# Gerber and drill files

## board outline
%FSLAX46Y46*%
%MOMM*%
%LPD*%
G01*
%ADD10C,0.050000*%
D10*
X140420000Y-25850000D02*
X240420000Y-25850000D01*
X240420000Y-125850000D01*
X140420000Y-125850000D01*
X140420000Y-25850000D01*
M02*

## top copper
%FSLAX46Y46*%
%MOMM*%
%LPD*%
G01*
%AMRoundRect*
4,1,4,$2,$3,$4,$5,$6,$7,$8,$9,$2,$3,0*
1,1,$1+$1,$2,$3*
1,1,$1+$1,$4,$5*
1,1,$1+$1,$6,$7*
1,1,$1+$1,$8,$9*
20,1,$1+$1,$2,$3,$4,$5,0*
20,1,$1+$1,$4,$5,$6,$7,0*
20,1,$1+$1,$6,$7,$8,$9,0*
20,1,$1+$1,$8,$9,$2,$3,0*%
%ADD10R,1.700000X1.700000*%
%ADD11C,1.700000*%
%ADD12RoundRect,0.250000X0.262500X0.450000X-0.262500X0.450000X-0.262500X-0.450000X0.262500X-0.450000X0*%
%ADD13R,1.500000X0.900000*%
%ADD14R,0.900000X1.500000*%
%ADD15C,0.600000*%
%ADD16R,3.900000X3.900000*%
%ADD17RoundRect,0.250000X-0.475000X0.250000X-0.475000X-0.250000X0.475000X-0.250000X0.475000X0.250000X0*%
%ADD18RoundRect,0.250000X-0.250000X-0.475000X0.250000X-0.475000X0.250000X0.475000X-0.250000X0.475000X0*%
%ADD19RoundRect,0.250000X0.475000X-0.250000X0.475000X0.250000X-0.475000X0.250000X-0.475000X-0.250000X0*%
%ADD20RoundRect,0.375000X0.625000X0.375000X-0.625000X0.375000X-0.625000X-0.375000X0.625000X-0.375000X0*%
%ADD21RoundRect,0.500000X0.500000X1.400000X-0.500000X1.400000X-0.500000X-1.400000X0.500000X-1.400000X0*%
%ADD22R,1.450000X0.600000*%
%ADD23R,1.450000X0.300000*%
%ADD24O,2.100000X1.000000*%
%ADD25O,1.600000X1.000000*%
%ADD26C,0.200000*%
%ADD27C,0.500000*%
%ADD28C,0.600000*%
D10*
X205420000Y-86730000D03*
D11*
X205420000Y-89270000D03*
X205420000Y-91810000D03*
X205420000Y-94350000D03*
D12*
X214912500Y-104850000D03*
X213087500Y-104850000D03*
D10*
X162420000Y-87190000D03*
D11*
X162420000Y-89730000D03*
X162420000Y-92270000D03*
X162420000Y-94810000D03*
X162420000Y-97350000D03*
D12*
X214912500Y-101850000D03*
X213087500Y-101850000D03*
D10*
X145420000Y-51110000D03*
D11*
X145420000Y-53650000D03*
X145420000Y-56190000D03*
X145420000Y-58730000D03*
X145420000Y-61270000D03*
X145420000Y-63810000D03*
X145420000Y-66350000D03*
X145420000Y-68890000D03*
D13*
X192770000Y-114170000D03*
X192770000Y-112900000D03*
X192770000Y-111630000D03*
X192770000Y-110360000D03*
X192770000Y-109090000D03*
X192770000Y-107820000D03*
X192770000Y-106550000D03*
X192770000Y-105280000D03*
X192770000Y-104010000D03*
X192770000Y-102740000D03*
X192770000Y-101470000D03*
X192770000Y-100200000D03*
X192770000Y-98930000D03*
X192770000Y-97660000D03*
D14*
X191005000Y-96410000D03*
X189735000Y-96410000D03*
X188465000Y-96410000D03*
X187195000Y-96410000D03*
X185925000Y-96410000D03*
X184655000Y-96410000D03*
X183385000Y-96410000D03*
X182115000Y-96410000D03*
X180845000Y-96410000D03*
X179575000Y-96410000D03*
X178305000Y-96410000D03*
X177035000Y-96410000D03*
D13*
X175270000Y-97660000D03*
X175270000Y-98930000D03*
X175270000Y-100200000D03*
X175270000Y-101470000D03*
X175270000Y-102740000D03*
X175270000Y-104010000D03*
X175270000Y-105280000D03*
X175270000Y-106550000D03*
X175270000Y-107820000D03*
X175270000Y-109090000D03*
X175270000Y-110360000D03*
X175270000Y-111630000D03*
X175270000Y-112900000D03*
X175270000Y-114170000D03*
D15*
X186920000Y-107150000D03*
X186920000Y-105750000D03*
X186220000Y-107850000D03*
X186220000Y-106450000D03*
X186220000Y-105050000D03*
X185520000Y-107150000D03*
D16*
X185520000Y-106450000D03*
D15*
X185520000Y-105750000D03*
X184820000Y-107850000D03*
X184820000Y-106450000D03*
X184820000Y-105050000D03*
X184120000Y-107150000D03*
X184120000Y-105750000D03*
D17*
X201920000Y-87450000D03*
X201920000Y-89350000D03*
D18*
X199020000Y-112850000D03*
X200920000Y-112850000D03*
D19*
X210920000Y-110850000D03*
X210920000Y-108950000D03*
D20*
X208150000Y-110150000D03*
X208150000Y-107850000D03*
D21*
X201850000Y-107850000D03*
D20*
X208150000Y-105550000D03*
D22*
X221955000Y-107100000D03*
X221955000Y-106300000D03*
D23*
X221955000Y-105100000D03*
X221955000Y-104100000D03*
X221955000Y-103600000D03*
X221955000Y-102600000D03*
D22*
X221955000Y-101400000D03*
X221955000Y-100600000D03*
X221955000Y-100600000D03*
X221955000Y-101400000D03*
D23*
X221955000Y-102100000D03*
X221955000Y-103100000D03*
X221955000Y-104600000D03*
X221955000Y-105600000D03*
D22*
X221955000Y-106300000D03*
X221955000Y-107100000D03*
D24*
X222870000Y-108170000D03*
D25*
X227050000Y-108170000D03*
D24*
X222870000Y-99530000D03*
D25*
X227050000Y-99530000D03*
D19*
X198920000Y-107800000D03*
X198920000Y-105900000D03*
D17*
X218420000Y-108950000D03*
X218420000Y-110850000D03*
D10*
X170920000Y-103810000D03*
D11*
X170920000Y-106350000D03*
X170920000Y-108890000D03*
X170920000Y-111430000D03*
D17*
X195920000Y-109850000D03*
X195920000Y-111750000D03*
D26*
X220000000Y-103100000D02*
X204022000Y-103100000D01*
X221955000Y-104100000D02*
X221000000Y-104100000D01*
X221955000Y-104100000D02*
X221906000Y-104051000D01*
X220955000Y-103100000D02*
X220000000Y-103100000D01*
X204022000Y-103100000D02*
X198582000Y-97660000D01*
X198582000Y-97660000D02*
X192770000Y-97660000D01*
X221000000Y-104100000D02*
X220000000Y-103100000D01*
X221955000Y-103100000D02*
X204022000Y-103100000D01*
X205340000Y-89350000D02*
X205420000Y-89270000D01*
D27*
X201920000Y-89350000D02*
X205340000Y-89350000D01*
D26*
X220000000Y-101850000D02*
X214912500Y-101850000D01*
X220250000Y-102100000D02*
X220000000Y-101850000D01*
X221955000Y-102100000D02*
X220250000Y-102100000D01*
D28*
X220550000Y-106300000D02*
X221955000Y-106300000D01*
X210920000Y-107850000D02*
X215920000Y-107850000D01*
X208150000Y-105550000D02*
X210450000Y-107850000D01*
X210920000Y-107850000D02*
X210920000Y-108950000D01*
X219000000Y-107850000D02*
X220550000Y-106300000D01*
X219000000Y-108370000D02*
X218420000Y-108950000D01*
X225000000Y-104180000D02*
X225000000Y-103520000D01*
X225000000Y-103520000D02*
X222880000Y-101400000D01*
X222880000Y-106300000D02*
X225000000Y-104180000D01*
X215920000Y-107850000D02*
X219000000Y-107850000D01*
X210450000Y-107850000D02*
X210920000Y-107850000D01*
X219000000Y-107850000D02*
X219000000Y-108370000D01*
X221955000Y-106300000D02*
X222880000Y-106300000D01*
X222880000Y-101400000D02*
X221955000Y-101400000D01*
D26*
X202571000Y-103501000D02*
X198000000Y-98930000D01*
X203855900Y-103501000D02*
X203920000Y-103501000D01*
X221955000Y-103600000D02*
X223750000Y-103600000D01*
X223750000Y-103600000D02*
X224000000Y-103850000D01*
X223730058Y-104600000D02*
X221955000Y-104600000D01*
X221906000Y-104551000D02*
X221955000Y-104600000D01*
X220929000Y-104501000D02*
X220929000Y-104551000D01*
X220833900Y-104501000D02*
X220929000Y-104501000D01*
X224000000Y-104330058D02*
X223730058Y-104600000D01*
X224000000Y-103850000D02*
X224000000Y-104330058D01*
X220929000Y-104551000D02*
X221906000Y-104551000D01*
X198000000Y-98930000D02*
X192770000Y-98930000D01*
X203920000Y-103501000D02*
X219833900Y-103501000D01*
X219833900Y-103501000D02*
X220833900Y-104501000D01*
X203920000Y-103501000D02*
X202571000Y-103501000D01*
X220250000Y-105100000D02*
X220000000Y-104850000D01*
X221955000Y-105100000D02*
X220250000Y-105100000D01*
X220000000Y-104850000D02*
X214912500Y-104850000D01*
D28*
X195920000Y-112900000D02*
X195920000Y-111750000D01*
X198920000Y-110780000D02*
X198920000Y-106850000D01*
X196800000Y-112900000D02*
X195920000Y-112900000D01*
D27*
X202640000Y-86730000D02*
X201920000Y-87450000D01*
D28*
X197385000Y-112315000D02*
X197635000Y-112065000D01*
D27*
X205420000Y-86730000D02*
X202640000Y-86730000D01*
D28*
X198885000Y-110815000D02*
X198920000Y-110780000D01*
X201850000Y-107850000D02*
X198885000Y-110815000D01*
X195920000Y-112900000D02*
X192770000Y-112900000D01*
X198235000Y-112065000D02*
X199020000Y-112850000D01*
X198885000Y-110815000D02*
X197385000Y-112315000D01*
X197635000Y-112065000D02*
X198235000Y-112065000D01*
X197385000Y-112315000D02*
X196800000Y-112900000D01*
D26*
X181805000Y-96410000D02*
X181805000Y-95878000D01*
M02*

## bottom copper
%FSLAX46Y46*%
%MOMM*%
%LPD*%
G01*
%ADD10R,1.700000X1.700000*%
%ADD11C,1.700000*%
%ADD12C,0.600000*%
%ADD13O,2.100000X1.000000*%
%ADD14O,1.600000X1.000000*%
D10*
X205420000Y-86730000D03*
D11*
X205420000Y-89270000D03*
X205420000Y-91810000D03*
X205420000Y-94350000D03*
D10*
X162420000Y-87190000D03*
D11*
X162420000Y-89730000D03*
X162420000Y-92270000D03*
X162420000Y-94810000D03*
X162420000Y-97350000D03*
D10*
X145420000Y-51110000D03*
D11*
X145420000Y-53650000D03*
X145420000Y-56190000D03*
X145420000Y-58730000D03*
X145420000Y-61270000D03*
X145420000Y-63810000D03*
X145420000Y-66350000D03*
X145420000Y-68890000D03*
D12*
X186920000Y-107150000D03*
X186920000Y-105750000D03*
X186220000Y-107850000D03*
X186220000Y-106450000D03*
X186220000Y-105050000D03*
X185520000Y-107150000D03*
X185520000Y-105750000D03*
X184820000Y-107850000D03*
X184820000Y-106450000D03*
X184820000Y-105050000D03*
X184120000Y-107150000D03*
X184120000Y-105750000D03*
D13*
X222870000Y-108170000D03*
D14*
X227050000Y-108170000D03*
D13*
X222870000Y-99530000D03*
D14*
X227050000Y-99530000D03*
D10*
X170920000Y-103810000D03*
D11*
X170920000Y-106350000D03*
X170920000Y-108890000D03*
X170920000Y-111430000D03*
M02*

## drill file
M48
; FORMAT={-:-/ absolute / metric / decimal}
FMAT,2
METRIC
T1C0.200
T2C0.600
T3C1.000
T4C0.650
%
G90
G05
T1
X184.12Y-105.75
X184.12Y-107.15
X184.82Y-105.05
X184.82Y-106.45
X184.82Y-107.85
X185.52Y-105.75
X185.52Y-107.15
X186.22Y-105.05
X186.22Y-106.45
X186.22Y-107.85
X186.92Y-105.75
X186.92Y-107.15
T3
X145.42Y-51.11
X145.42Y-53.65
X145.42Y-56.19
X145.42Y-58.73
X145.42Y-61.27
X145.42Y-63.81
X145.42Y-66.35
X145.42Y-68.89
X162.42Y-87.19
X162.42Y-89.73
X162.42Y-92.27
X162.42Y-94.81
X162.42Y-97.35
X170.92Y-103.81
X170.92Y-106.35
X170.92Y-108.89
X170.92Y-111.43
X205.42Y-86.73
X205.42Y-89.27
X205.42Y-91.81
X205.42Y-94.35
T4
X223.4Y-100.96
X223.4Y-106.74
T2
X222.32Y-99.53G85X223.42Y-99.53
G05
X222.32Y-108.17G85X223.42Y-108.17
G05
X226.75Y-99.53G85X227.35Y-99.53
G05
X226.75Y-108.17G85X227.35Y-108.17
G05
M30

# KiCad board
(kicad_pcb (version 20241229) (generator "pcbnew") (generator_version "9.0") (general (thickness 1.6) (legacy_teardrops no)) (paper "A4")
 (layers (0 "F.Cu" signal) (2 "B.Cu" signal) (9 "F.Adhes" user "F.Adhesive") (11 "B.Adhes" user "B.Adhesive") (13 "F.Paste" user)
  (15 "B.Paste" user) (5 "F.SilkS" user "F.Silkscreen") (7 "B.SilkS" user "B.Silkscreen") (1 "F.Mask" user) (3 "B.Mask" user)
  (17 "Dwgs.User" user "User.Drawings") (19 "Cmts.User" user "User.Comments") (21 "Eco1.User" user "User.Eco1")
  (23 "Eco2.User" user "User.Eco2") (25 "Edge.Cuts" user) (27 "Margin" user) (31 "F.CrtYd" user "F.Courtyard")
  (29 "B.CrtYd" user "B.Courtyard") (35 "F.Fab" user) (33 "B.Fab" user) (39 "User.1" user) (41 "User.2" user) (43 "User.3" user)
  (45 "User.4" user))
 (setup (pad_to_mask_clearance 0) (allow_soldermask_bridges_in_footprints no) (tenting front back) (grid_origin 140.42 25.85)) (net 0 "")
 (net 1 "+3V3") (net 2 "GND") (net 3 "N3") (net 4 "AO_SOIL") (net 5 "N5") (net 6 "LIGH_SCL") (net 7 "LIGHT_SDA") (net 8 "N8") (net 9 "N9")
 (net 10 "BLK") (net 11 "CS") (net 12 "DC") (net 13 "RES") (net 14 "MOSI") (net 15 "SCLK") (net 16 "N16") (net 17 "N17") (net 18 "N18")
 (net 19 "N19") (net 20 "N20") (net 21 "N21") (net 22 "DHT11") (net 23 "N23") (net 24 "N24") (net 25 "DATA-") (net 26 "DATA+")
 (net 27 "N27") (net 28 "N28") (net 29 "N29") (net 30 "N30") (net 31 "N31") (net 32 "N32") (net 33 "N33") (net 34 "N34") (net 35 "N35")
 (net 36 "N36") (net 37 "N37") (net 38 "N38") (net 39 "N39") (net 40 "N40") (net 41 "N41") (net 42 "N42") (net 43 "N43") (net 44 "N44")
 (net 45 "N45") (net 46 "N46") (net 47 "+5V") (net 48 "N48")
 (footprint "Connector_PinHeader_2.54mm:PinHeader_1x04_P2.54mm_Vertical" (layer "F.Cu") (at 205.42 86.73)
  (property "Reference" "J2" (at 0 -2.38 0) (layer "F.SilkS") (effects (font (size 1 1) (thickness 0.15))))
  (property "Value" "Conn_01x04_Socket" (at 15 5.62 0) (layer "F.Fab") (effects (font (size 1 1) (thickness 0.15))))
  (pad "1" thru_hole rect (at 0 0) (size 1.7 1.7) (drill 1) (layers "*.Cu" "*.Mask") (remove_unused_layers no) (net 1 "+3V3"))
  (pad "2" thru_hole circle (at 0 2.54) (size 1.7 1.7) (drill 1) (layers "*.Cu" "*.Mask") (remove_unused_layers no) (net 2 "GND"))
  (pad "3" thru_hole circle (at 0 5.08) (size 1.7 1.7) (drill 1) (layers "*.Cu" "*.Mask") (remove_unused_layers no) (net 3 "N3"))
  (pad "4" thru_hole circle (at 0 7.62) (size 1.7 1.7) (drill 1) (layers "*.Cu" "*.Mask") (remove_unused_layers no) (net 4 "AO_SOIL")))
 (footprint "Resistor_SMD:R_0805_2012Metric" (layer "F.Cu") (at 214 104.85 180)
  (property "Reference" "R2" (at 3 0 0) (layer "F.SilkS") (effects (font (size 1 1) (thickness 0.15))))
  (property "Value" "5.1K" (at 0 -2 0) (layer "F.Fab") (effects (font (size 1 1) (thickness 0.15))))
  (pad "1" smd roundrect (at -0.9125 0 180) (size 1.025 1.4) (layers "F.Cu" "F.Mask" "F.Paste") (roundrect_rratio 0.243902) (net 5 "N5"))
  (pad "2" smd roundrect (at 0.9125 0 180) (size 1.025 1.4) (layers "F.Cu" "F.Mask" "F.Paste") (roundrect_rratio 0.243902) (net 2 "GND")))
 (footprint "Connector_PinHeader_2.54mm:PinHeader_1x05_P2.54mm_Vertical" (layer "F.Cu") (at 162.42 87.19)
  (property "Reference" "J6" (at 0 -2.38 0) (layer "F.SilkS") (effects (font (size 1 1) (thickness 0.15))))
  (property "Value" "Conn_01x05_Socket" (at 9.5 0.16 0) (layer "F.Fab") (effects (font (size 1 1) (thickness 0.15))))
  (pad "1" thru_hole rect (at 0 0) (size 1.7 1.7) (drill 1) (layers "*.Cu" "*.Mask") (remove_unused_layers no) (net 1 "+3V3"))
  (pad "2" thru_hole circle (at 0 2.54) (size 1.7 1.7) (drill 1) (layers "*.Cu" "*.Mask") (remove_unused_layers no) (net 2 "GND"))
  (pad "3" thru_hole circle (at 0 5.08) (size 1.7 1.7) (drill 1) (layers "*.Cu" "*.Mask") (remove_unused_layers no) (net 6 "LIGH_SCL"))
  (pad "4" thru_hole circle (at 0 7.62) (size 1.7 1.7) (drill 1) (layers "*.Cu" "*.Mask") (remove_unused_layers no) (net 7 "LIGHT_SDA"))
  (pad "5" thru_hole circle (at 0 10.16) (size 1.7 1.7) (drill 1) (layers "*.Cu" "*.Mask") (remove_unused_layers no) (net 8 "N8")))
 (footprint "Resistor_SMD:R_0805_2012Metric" (layer "F.Cu") (at 214 101.85 180)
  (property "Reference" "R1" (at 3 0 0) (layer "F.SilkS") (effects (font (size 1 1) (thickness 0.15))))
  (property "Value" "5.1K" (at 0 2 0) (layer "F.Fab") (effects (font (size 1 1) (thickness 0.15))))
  (pad "1" smd roundrect (at -0.9125 0 180) (size 1.025 1.4) (layers "F.Cu" "F.Mask" "F.Paste") (roundrect_rratio 0.243902) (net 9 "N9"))
  (pad "2" smd roundrect (at 0.9125 0 180) (size 1.025 1.4) (layers "F.Cu" "F.Mask" "F.Paste") (roundrect_rratio 0.243902) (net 2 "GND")))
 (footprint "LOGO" (layer "F.Cu") (at 224.5 115)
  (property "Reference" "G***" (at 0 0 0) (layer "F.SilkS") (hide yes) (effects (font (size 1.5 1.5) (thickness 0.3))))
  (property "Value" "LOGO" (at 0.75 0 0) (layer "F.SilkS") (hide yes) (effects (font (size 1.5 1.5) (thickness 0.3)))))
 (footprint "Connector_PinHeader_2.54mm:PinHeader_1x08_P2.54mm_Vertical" (layer "F.Cu") (at 145.42 51.11)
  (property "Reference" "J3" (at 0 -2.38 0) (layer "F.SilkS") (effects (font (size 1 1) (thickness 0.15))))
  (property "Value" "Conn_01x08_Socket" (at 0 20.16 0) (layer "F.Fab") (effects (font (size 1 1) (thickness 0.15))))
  (pad "1" thru_hole rect (at 0 0) (size 1.7 1.7) (drill 1) (layers "*.Cu" "*.Mask") (remove_unused_layers no) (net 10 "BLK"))
  (pad "2" thru_hole circle (at 0 2.54) (size 1.7 1.7) (drill 1) (layers "*.Cu" "*.Mask") (remove_unused_layers no) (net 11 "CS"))
  (pad "3" thru_hole circle (at 0 5.08) (size 1.7 1.7) (drill 1) (layers "*.Cu" "*.Mask") (remove_unused_layers no) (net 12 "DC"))
  (pad "4" thru_hole circle (at 0 7.62) (size 1.7 1.7) (drill 1) (layers "*.Cu" "*.Mask") (remove_unused_layers no) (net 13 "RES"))
  (pad "5" thru_hole circle (at 0 10.16) (size 1.7 1.7) (drill 1) (layers "*.Cu" "*.Mask") (remove_unused_layers no) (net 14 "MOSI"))
  (pad "6" thru_hole circle (at 0 12.7) (size 1.7 1.7) (drill 1) (layers "*.Cu" "*.Mask") (remove_unused_layers no) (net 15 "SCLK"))
  (pad "7" thru_hole circle (at 0 15.24) (size 1.7 1.7) (drill 1) (layers "*.Cu" "*.Mask") (remove_unused_layers no) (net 1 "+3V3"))
  (pad "8" thru_hole circle (at 0 17.78) (size 1.7 1.7) (drill 1) (layers "*.Cu" "*.Mask") (remove_unused_layers no) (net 2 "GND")))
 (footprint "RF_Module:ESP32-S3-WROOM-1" (layer "F.Cu") (at 184.02 108.91 180)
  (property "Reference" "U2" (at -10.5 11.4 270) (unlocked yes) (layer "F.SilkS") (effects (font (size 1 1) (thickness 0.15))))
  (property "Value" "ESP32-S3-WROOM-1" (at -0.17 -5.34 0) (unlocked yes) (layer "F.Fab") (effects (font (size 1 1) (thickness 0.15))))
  (pad "" smd rect (at -2.9 1.06 180) (size 0.9 0.9) (layers "F.Paste"))
  (pad "" smd rect (at -2.9 2.46 90) (size 0.9 0.9) (layers "F.Paste"))
  (pad "" smd rect (at -2.9 3.86 180) (size 0.9 0.9) (layers "F.Paste"))
  (pad "" smd rect (at -1.5 1.06 90) (size 0.9 0.9) (layers "F.Paste"))
  (pad "" smd rect (at -1.5 2.46 90) (size 0.9 0.9) (layers "F.Paste"))
  (pad "" smd rect (at -1.5 3.86 90) (size 0.9 0.9) (layers "F.Paste"))
  (pad "" smd rect (at -0.1 1.06 90) (size 0.9 0.9) (layers "F.Paste"))
  (pad "" smd rect (at -0.1 2.46 90) (size 0.9 0.9) (layers "F.Paste"))
  (pad "" smd rect (at -0.1 3.86 90) (size 0.9 0.9) (layers "F.Paste"))
  (pad "1" smd rect (at -8.75 -5.26 180) (size 1.5 0.9) (layers "F.Cu" "F.Mask" "F.Paste") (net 2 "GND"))
  (pad "2" smd rect (at -8.75 -3.99 180) (size 1.5 0.9) (layers "F.Cu" "F.Mask" "F.Paste") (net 1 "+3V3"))
  (pad "3" smd rect (at -8.75 -2.72 180) (size 1.5 0.9) (layers "F.Cu" "F.Mask" "F.Paste") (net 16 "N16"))
  (pad "4" smd rect (at -8.75 -1.45 180) (size 1.5 0.9) (layers "F.Cu" "F.Mask" "F.Paste") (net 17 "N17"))
  (pad "5" smd rect (at -8.75 -0.18 180) (size 1.5 0.9) (layers "F.Cu" "F.Mask" "F.Paste") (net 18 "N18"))
  (pad "6" smd rect (at -8.75 1.09 180) (size 1.5 0.9) (layers "F.Cu" "F.Mask" "F.Paste") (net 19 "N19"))
  (pad "7" smd rect (at -8.75 2.36 180) (size 1.5 0.9) (layers "F.Cu" "F.Mask" "F.Paste") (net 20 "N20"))
  (pad "8" smd rect (at -8.75 3.63 180) (size 1.5 0.9) (layers "F.Cu" "F.Mask" "F.Paste") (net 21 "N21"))
  (pad "9" smd rect (at -8.75 4.9 180) (size 1.5 0.9) (layers "F.Cu" "F.Mask" "F.Paste") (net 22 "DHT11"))
  (pad "10" smd rect (at -8.75 6.17 180) (size 1.5 0.9) (layers "F.Cu" "F.Mask" "F.Paste") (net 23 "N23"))
  (pad "11" smd rect (at -8.75 7.44 180) (size 1.5 0.9) (layers "F.Cu" "F.Mask" "F.Paste") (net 4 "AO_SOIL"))
  (pad "12" smd rect (at -8.75 8.71 180) (size 1.5 0.9) (layers "F.Cu" "F.Mask" "F.Paste") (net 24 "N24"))
  (pad "13" smd rect (at -8.75 9.98 180) (size 1.5 0.9) (layers "F.Cu" "F.Mask" "F.Paste") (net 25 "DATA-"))
  (pad "14" smd rect (at -8.75 11.25) (size 1.5 0.9) (layers "F.Cu" "F.Mask" "F.Paste") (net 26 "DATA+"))
  (pad "15" smd rect (at -6.985 12.5 90) (size 1.5 0.9) (layers "F.Cu" "F.Mask" "F.Paste") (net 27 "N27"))
  (pad "16" smd rect (at -5.715 12.5 90) (size 1.5 0.9) (layers "F.Cu" "F.Mask" "F.Paste") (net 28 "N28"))
  (pad "17" smd rect (at -4.445 12.5 90) (size 1.5 0.9) (layers "F.Cu" "F.Mask" "F.Paste") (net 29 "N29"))
  (pad "18" smd rect (at -3.175 12.5 90) (size 1.5 0.9) (layers "F.Cu" "F.Mask" "F.Paste") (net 11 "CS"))
  (pad "19" smd rect (at -1.905 12.5 90) (size 1.5 0.9) (layers "F.Cu" "F.Mask" "F.Paste") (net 14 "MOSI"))
  (pad "20" smd rect (at -0.635 12.5 90) (size 1.5 0.9) (layers "F.Cu" "F.Mask" "F.Paste") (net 15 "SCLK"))
  (pad "21" smd rect (at 0.635 12.5 90) (size 1.5 0.9) (layers "F.Cu" "F.Mask" "F.Paste") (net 13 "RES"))
  (pad "22" smd rect (at 1.905 12.5 90) (size 1.5 0.9) (layers "F.Cu" "F.Mask" "F.Paste") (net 12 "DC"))
  (pad "23" smd rect (at 3.175 12.5 90) (size 1.5 0.9) (layers "F.Cu" "F.Mask" "F.Paste") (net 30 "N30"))
  (pad "24" smd rect (at 4.445 12.5 90) (size 1.5 0.9) (layers "F.Cu" "F.Mask" "F.Paste") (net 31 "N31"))
  (pad "25" smd rect (at 5.715 12.5 90) (size 1.5 0.9) (layers "F.Cu" "F.Mask" "F.Paste") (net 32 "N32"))
  (pad "26" smd rect (at 6.985 12.5 90) (size 1.5 0.9) (layers "F.Cu" "F.Mask" "F.Paste") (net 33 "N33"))
  (pad "27" smd rect (at 8.75 11.25 180) (size 1.5 0.9) (layers "F.Cu" "F.Mask" "F.Paste") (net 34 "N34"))
  (pad "28" smd rect (at 8.75 9.98 180) (size 1.5 0.9) (layers "F.Cu" "F.Mask" "F.Paste") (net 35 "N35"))
  (pad "29" smd rect (at 8.75 8.71 180) (size 1.5 0.9) (layers "F.Cu" "F.Mask" "F.Paste") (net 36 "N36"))
  (pad "30" smd rect (at 8.75 7.44 180) (size 1.5 0.9) (layers "F.Cu" "F.Mask" "F.Paste") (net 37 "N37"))
  (pad "31" smd rect (at 8.75 6.17 180) (size 1.5 0.9) (layers "F.Cu" "F.Mask" "F.Paste") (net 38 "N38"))
  (pad "32" smd rect (at 8.75 4.9 180) (size 1.5 0.9) (layers "F.Cu" "F.Mask" "F.Paste") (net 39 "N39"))
  (pad "33" smd rect (at 8.75 3.63 180) (size 1.5 0.9) (layers "F.Cu" "F.Mask" "F.Paste") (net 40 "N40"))
  (pad "34" smd rect (at 8.75 2.36 180) (size 1.5 0.9) (layers "F.Cu" "F.Mask" "F.Paste") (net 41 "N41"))
  (pad "35" smd rect (at 8.75 1.09 180) (size 1.5 0.9) (layers "F.Cu" "F.Mask" "F.Paste") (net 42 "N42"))
  (pad "36" smd rect (at 8.75 -0.18 180) (size 1.5 0.9) (layers "F.Cu" "F.Mask" "F.Paste") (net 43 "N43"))
  (pad "37" smd rect (at 8.75 -1.45 180) (size 1.5 0.9) (layers "F.Cu" "F.Mask" "F.Paste") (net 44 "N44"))
  (pad "38" smd rect (at 8.75 -2.72 180) (size 1.5 0.9) (layers "F.Cu" "F.Mask" "F.Paste") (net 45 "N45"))
  (pad "39" smd rect (at 8.75 -3.99 180) (size 1.5 0.9) (layers "F.Cu" "F.Mask" "F.Paste") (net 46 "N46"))
  (pad "40" smd rect (at 8.75 -5.26 180) (size 1.5 0.9) (layers "F.Cu" "F.Mask" "F.Paste") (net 2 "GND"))
  (pad "41" thru_hole circle (at -2.9 1.76 270) (size 0.6 0.6) (drill 0.2) (layers "*.Cu" "F.Mask") (remove_unused_layers no) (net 2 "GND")
   (zone_connect 2))
  (pad "41" thru_hole circle (at -2.9 3.16 180) (size 0.6 0.6) (drill 0.2) (layers "*.Cu" "F.Mask") (remove_unused_layers no) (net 2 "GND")
   (zone_connect 2))
  (pad "41" thru_hole circle (at -2.2 1.06 180) (size 0.6 0.6) (drill 0.2) (layers "*.Cu" "F.Mask") (remove_unused_layers no) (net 2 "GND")
   (zone_connect 2))
  (pad "41" thru_hole circle (at -2.2 2.46 180) (size 0.6 0.6) (drill 0.2) (layers "*.Cu" "F.Mask") (remove_unused_layers no) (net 2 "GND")
   (zone_connect 2))
  (pad "41" thru_hole circle (at -2.2 3.86 180) (size 0.6 0.6) (drill 0.2) (layers "*.Cu" "F.Mask") (remove_unused_layers no) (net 2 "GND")
   (zone_connect 2))
  (pad "41" thru_hole circle (at -1.5 1.76 180) (size 0.6 0.6) (drill 0.2) (layers "*.Cu" "F.Mask") (remove_unused_layers no) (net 2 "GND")
   (zone_connect 2))
  (pad "41" smd rect (at -1.5 2.46 90) (size 3.9 3.9) (layers "F.Cu" "F.Mask") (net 2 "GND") (zone_connect 2))
  (pad "41" thru_hole circle (at -1.5 3.16 180) (size 0.6 0.6) (drill 0.2) (layers "*.Cu" "F.Mask") (remove_unused_layers no) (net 2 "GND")
   (zone_connect 2))
  (pad "41" thru_hole circle (at -0.8 1.06 180) (size 0.6 0.6) (drill 0.2) (layers "*.Cu" "F.Mask") (remove_unused_layers no) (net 2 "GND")
   (zone_connect 2))
  (pad "41" thru_hole circle (at -0.8 2.46 180) (size 0.6 0.6) (drill 0.2) (layers "*.Cu" "F.Mask") (remove_unused_layers no) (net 2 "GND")
   (zone_connect 2))
  (pad "41" thru_hole circle (at -0.8 3.86 180) (size 0.6 0.6) (drill 0.2) (layers "*.Cu" "F.Mask") (remove_unused_layers no) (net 2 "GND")
   (zone_connect 2))
  (pad "41" thru_hole circle (at -0.1 1.76 180) (size 0.6 0.6) (drill 0.2) (layers "*.Cu" "F.Mask") (remove_unused_layers no) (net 2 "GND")
   (zone_connect 2))
  (pad "41" thru_hole circle (at -0.1 3.16 180) (size 0.6 0.6) (drill 0.2) (layers "*.Cu" "F.Mask") (remove_unused_layers no) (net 2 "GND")
   (zone_connect 2))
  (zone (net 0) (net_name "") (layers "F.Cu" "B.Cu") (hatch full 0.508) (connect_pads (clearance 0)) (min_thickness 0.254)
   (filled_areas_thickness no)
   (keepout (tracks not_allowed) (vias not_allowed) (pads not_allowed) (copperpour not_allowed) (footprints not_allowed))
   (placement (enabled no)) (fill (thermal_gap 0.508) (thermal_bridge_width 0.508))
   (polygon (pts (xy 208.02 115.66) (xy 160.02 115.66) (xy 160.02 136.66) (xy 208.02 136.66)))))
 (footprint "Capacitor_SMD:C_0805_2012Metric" (layer "F.Cu") (at 201.92 88.4 -90)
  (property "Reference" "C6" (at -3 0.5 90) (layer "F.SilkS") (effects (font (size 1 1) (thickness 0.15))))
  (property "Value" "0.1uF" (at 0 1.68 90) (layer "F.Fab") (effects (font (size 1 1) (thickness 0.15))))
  (pad "1" smd roundrect (at -0.95 0 270) (size 1 1.45) (layers "F.Cu" "F.Mask" "F.Paste") (roundrect_rratio 0.25) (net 1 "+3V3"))
  (pad "2" smd roundrect (at 0.95 0 270) (size 1 1.45) (layers "F.Cu" "F.Mask" "F.Paste") (roundrect_rratio 0.25) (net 2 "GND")))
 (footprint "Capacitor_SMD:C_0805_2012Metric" (layer "F.Cu") (at 199.97 112.85)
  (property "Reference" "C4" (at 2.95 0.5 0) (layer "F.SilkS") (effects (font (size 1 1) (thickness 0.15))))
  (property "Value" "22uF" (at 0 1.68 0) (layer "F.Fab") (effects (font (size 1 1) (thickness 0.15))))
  (pad "1" smd roundrect (at -0.95 0) (size 1 1.45) (layers "F.Cu" "F.Mask" "F.Paste") (roundrect_rratio 0.25) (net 1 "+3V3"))
  (pad "2" smd roundrect (at 0.95 0) (size 1 1.45) (layers "F.Cu" "F.Mask" "F.Paste") (roundrect_rratio 0.25) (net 2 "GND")))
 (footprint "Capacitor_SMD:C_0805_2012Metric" (layer "F.Cu") (at 210.92 109.9 90)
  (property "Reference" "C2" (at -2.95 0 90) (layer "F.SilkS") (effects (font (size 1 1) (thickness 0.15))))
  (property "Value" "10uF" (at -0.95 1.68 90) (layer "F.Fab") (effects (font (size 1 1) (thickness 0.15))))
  (pad "1" smd roundrect (at -0.95 0 90) (size 1 1.45) (layers "F.Cu" "F.Mask" "F.Paste") (roundrect_rratio 0.25) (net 2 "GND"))
  (pad "2" smd roundrect (at 0.95 0 90) (size 1 1.45) (layers "F.Cu" "F.Mask" "F.Paste") (roundrect_rratio 0.25) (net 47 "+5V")))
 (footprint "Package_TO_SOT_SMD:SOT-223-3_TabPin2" (layer "F.Cu") (at 205 107.85 180)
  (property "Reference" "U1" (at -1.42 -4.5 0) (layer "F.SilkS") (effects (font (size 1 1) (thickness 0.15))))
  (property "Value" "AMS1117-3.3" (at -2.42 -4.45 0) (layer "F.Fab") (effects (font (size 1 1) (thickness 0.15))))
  (pad "1" smd roundrect (at -3.15 -2.3 180) (size 2 1.5) (layers "F.Cu" "F.Mask" "F.Paste") (roundrect_rratio 0.25) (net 2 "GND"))
  (pad "2" smd roundrect (at -3.15 0 180) (size 2 1.5) (layers "F.Cu" "F.Mask" "F.Paste") (roundrect_rratio 0.25) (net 1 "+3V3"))
  (pad "2" smd roundrect (at 3.15 0 180) (size 2 3.8) (layers "F.Cu" "F.Mask" "F.Paste") (roundrect_rratio 0.25) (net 1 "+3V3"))
  (pad "3" smd roundrect (at -3.15 2.3 180) (size 2 1.5) (layers "F.Cu" "F.Mask" "F.Paste") (roundrect_rratio 0.25) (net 47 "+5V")))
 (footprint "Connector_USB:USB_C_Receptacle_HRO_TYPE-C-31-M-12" (layer "F.Cu") (at 226 103.85 90)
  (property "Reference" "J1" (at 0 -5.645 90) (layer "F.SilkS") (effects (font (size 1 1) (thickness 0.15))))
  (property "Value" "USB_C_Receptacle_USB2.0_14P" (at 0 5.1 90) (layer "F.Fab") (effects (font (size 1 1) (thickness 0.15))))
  (pad "" np_thru_hole circle (at -2.89 -2.6 90) (size 0.65 0.65) (drill 0.65) (layers "*.Cu" "*.Mask"))
  (pad "" np_thru_hole circle (at 2.89 -2.6 90) (size 0.65 0.65) (drill 0.65) (layers "*.Cu" "*.Mask"))
  (pad "A1" smd rect (at -3.25 -4.045 90) (size 0.6 1.45) (layers "F.Cu" "F.Mask" "F.Paste") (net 2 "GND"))
  (pad "A4" smd rect (at -2.45 -4.045 90) (size 0.6 1.45) (layers "F.Cu" "F.Mask" "F.Paste") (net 47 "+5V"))
  (pad "A5" smd rect (at -1.25 -4.045 90) (size 0.3 1.45) (layers "F.Cu" "F.Mask" "F.Paste") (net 5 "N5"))
  (pad "A6" smd rect (at -0.25 -4.045 90) (size 0.3 1.45) (layers "F.Cu" "F.Mask" "F.Paste") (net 26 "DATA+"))
  (pad "A7" smd rect (at 0.25 -4.045 90) (size 0.3 1.45) (layers "F.Cu" "F.Mask" "F.Paste") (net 25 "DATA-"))
  (pad "A8" smd rect (at 1.25 -4.045 90) (size 0.3 1.45) (layers "F.Cu" "F.Mask" "F.Paste"))
  (pad "A9" smd rect (at 2.45 -4.045 90) (size 0.6 1.45) (layers "F.Cu" "F.Mask" "F.Paste") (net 47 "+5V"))
  (pad "A12" smd rect (at 3.25 -4.045 90) (size 0.6 1.45) (layers "F.Cu" "F.Mask" "F.Paste") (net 2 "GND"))
  (pad "B1" smd rect (at 3.25 -4.045 90) (size 0.6 1.45) (layers "F.Cu" "F.Mask" "F.Paste") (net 2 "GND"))
  (pad "B4" smd rect (at 2.45 -4.045 90) (size 0.6 1.45) (layers "F.Cu" "F.Mask" "F.Paste") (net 47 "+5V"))
  (pad "B5" smd rect (at 1.75 -4.045 90) (size 0.3 1.45) (layers "F.Cu" "F.Mask" "F.Paste") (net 9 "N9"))
  (pad "B6" smd rect (at 0.75 -4.045 90) (size 0.3 1.45) (layers "F.Cu" "F.Mask" "F.Paste") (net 26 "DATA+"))
  (pad "B7" smd rect (at -0.75 -4.045 90) (size 0.3 1.45) (layers "F.Cu" "F.Mask" "F.Paste") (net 25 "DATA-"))
  (pad "B8" smd rect (at -1.75 -4.045 90) (size 0.3 1.45) (layers "F.Cu" "F.Mask" "F.Paste"))
  (pad "B9" smd rect (at -2.45 -4.045 90) (size 0.6 1.45) (layers "F.Cu" "F.Mask" "F.Paste") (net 47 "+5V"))
  (pad "B12" smd rect (at -3.25 -4.045 90) (size 0.6 1.45) (layers "F.Cu" "F.Mask" "F.Paste") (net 2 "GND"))
  (pad "S1" thru_hole oval (at -4.32 -3.13 90) (size 1 2.1) (drill oval 0.6 1.7) (layers "*.Cu" "*.Mask") (remove_unused_layers no)
   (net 2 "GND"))
  (pad "S1" thru_hole oval (at -4.32 1.05 90) (size 1 1.6) (drill oval 0.6 1.2) (layers "*.Cu" "*.Mask") (remove_unused_layers no)
   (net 2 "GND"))
  (pad "S1" thru_hole oval (at 4.32 -3.13 90) (size 1 2.1) (drill oval 0.6 1.7) (layers "*.Cu" "*.Mask") (remove_unused_layers no)
   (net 2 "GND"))
  (pad "S1" thru_hole oval (at 4.32 1.05 90) (size 1 1.6) (drill oval 0.6 1.2) (layers "*.Cu" "*.Mask") (remove_unused_layers no)
   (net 2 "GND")))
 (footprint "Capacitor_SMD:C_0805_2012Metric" (layer "F.Cu") (at 198.92 106.85 90)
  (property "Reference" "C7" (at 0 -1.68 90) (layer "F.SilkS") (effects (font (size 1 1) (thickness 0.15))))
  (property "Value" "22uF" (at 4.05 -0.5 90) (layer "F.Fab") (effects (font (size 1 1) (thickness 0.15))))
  (pad "1" smd roundrect (at -0.95 0 90) (size 1 1.45) (layers "F.Cu" "F.Mask" "F.Paste") (roundrect_rratio 0.25) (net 1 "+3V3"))
  (pad "2" smd roundrect (at 0.95 0 90) (size 1 1.45) (layers "F.Cu" "F.Mask" "F.Paste") (roundrect_rratio 0.25) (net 2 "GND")))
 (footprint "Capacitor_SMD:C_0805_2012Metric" (layer "F.Cu") (at 218.42 109.9 -90)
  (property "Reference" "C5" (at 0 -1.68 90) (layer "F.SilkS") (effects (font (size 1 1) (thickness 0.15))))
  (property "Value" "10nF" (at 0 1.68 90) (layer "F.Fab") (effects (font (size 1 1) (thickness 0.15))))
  (pad "1" smd roundrect (at -0.95 0 270) (size 1 1.45) (layers "F.Cu" "F.Mask" "F.Paste") (roundrect_rratio 0.25) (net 47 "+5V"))
  (pad "2" smd roundrect (at 0.95 0 270) (size 1 1.45) (layers "F.Cu" "F.Mask" "F.Paste") (roundrect_rratio 0.25) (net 2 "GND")))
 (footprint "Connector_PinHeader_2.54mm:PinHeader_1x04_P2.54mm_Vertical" (layer "F.Cu") (at 170.92 103.81)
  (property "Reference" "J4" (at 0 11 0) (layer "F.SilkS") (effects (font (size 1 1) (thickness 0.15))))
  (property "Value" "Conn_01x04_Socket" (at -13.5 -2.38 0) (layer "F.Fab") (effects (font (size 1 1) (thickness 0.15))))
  (pad "1" thru_hole rect (at 0 0) (size 1.7 1.7) (drill 1) (layers "*.Cu" "*.Mask") (remove_unused_layers no) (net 1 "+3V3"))
  (pad "2" thru_hole circle (at 0 2.54) (size 1.7 1.7) (drill 1) (layers "*.Cu" "*.Mask") (remove_unused_layers no) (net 22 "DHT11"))
  (pad "3" thru_hole circle (at 0 5.08) (size 1.7 1.7) (drill 1) (layers "*.Cu" "*.Mask") (remove_unused_layers no) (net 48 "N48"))
  (pad "4" thru_hole circle (at 0 7.62) (size 1.7 1.7) (drill 1) (layers "*.Cu" "*.Mask") (remove_unused_layers no) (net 2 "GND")))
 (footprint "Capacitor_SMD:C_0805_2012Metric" (layer "F.Cu") (at 195.92 110.8 -90)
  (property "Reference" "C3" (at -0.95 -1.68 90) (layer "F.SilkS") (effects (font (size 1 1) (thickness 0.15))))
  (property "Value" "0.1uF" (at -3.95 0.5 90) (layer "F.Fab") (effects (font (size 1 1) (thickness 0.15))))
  (pad "1" smd roundrect (at -0.95 0 270) (size 1 1.45) (layers "F.Cu" "F.Mask" "F.Paste") (roundrect_rratio 0.25) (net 2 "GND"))
  (pad "2" smd roundrect (at 0.95 0 270) (size 1 1.45) (layers "F.Cu" "F.Mask" "F.Paste") (roundrect_rratio 0.25) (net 1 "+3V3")))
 (gr_rect (start 140.42 25.85) (end 240.42 125.85) (stroke (width 0.05) (type solid)) (fill no) (layer "Edge.Cuts"))
 (segment (start 220 103.1) (end 204.022 103.1) (width 0.2) (layer "F.Cu") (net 26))
 (segment (start 221.955 104.1) (end 221 104.1) (width 0.2) (layer "F.Cu") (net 26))
 (segment (start 221.955 104.1) (end 221.906 104.051) (width 0.2) (layer "F.Cu") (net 26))
 (segment (start 220.955 103.1) (end 220 103.1) (width 0.2) (layer "F.Cu") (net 26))
 (segment (start 204.022 103.1) (end 198.582 97.66) (width 0.2) (layer "F.Cu") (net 26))
 (segment (start 198.582 97.66) (end 192.77 97.66) (width 0.2) (layer "F.Cu") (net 26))
 (segment (start 221 104.1) (end 220 103.1) (width 0.2) (layer "F.Cu") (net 26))
 (segment (start 221.955 103.1) (end 204.022 103.1) (width 0.2) (layer "F.Cu") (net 26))
 (segment (start 205.34 89.35) (end 205.42 89.27) (width 0.2) (layer "F.Cu") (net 2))
 (segment (start 201.92 89.35) (end 205.34 89.35) (width 0.5) (layer "F.Cu") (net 2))
 (segment (start 220 101.85) (end 214.9125 101.85) (width 0.2) (layer "F.Cu") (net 9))
 (segment (start 220.25 102.1) (end 220 101.85) (width 0.2) (layer "F.Cu") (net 9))
 (segment (start 221.955 102.1) (end 220.25 102.1) (width 0.2) (layer "F.Cu") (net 9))
 (segment (start 220.55 106.3) (end 221.955 106.3) (width 0.6) (layer "F.Cu") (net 47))
 (segment (start 210.92 107.85) (end 215.92 107.85) (width 0.6) (layer "F.Cu") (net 47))
 (segment (start 208.15 105.55) (end 210.45 107.85) (width 0.6) (layer "F.Cu") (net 47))
 (segment (start 210.92 107.85) (end 210.92 108.95) (width 0.6) (layer "F.Cu") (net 47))
 (segment (start 219 107.85) (end 220.55 106.3) (width 0.6) (layer "F.Cu") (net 47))
 (segment (start 219 108.37) (end 218.42 108.95) (width 0.6) (layer "F.Cu") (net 47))
 (segment (start 225 104.18) (end 225 103.52) (width 0.6) (layer "F.Cu") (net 47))
 (segment (start 225 103.52) (end 222.88 101.4) (width 0.6) (layer "F.Cu") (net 47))
 (segment (start 222.88 106.3) (end 225 104.18) (width 0.6) (layer "F.Cu") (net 47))
 (segment (start 215.92 107.85) (end 219 107.85) (width 0.6) (layer "F.Cu") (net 47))
 (segment (start 210.45 107.85) (end 210.92 107.85) (width 0.6) (layer "F.Cu") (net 47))
 (segment (start 219 107.85) (end 219 108.37) (width 0.6) (layer "F.Cu") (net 47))
 (segment (start 221.955 106.3) (end 222.88 106.3) (width 0.6) (layer "F.Cu") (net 47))
 (segment (start 222.88 101.4) (end 221.955 101.4) (width 0.6) (layer "F.Cu") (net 47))
 (segment (start 202.571 103.501) (end 198 98.93) (width 0.2) (layer "F.Cu") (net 25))
 (segment (start 203.8559 103.501) (end 203.92 103.501) (width 0.2) (layer "F.Cu") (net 25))
 (segment (start 221.955 103.6) (end 223.75 103.6) (width 0.2) (layer "F.Cu") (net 25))
 (segment (start 223.75 103.6) (end 224 103.85) (width 0.2) (layer "F.Cu") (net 25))
 (segment (start 223.730058 104.6) (end 221.955 104.6) (width 0.2) (layer "F.Cu") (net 25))
 (segment (start 221.906 104.551) (end 221.955 104.6) (width 0.2) (layer "F.Cu") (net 25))
 (segment (start 220.929 104.501) (end 220.929 104.551) (width 0.2) (layer "F.Cu") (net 25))
 (segment (start 220.8339 104.501) (end 220.929 104.501) (width 0.2) (layer "F.Cu") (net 25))
 (segment (start 224 104.330058) (end 223.730058 104.6) (width 0.2) (layer "F.Cu") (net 25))
 (segment (start 224 103.85) (end 224 104.330058) (width 0.2) (layer "F.Cu") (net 25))
 (segment (start 220.929 104.551) (end 221.906 104.551) (width 0.2) (layer "F.Cu") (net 25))
 (segment (start 198 98.93) (end 192.77 98.93) (width 0.2) (layer "F.Cu") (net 25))
 (segment (start 203.92 103.501) (end 219.8339 103.501) (width 0.2) (layer "F.Cu") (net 25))
 (segment (start 219.8339 103.501) (end 220.8339 104.501) (width 0.2) (layer "F.Cu") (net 25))
 (segment (start 203.92 103.501) (end 202.571 103.501) (width 0.2) (layer "F.Cu") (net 25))
 (segment (start 220.25 105.1) (end 220 104.85) (width 0.2) (layer "F.Cu") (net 5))
 (segment (start 221.955 105.1) (end 220.25 105.1) (width 0.2) (layer "F.Cu") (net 5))
 (segment (start 220 104.85) (end 214.9125 104.85) (width 0.2) (layer "F.Cu") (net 5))
 (segment (start 195.92 112.9) (end 195.92 111.75) (width 0.6) (layer "F.Cu") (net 1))
 (segment (start 198.92 110.78) (end 198.92 106.85) (width 0.6) (layer "F.Cu") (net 1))
 (segment (start 196.8 112.9) (end 195.92 112.9) (width 0.6) (layer "F.Cu") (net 1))
 (segment (start 202.64 86.73) (end 201.92 87.45) (width 0.5) (layer "F.Cu") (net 1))
 (segment (start 197.385 112.315) (end 197.635 112.065) (width 0.6) (layer "F.Cu") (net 1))
 (segment (start 205.42 86.73) (end 202.64 86.73) (width 0.5) (layer "F.Cu") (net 1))
 (segment (start 198.885 110.815) (end 198.92 110.78) (width 0.6) (layer "F.Cu") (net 1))
 (segment (start 201.85 107.85) (end 198.885 110.815) (width 0.6) (layer "F.Cu") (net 1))
 (segment (start 195.92 112.9) (end 192.77 112.9) (width 0.6) (layer "F.Cu") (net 1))
 (segment (start 198.235 112.065) (end 199.02 112.85) (width 0.6) (layer "F.Cu") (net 1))
 (segment (start 198.885 110.815) (end 197.385 112.315) (width 0.6) (layer "F.Cu") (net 1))
 (segment (start 197.635 112.065) (end 198.235 112.065) (width 0.6) (layer "F.Cu") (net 1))
 (segment (start 197.385 112.315) (end 196.8 112.9) (width 0.6) (layer "F.Cu") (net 1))
 (segment (start 181.805 96.41) (end 181.805 95.878) (width 0.2) (layer "F.Cu") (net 12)))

